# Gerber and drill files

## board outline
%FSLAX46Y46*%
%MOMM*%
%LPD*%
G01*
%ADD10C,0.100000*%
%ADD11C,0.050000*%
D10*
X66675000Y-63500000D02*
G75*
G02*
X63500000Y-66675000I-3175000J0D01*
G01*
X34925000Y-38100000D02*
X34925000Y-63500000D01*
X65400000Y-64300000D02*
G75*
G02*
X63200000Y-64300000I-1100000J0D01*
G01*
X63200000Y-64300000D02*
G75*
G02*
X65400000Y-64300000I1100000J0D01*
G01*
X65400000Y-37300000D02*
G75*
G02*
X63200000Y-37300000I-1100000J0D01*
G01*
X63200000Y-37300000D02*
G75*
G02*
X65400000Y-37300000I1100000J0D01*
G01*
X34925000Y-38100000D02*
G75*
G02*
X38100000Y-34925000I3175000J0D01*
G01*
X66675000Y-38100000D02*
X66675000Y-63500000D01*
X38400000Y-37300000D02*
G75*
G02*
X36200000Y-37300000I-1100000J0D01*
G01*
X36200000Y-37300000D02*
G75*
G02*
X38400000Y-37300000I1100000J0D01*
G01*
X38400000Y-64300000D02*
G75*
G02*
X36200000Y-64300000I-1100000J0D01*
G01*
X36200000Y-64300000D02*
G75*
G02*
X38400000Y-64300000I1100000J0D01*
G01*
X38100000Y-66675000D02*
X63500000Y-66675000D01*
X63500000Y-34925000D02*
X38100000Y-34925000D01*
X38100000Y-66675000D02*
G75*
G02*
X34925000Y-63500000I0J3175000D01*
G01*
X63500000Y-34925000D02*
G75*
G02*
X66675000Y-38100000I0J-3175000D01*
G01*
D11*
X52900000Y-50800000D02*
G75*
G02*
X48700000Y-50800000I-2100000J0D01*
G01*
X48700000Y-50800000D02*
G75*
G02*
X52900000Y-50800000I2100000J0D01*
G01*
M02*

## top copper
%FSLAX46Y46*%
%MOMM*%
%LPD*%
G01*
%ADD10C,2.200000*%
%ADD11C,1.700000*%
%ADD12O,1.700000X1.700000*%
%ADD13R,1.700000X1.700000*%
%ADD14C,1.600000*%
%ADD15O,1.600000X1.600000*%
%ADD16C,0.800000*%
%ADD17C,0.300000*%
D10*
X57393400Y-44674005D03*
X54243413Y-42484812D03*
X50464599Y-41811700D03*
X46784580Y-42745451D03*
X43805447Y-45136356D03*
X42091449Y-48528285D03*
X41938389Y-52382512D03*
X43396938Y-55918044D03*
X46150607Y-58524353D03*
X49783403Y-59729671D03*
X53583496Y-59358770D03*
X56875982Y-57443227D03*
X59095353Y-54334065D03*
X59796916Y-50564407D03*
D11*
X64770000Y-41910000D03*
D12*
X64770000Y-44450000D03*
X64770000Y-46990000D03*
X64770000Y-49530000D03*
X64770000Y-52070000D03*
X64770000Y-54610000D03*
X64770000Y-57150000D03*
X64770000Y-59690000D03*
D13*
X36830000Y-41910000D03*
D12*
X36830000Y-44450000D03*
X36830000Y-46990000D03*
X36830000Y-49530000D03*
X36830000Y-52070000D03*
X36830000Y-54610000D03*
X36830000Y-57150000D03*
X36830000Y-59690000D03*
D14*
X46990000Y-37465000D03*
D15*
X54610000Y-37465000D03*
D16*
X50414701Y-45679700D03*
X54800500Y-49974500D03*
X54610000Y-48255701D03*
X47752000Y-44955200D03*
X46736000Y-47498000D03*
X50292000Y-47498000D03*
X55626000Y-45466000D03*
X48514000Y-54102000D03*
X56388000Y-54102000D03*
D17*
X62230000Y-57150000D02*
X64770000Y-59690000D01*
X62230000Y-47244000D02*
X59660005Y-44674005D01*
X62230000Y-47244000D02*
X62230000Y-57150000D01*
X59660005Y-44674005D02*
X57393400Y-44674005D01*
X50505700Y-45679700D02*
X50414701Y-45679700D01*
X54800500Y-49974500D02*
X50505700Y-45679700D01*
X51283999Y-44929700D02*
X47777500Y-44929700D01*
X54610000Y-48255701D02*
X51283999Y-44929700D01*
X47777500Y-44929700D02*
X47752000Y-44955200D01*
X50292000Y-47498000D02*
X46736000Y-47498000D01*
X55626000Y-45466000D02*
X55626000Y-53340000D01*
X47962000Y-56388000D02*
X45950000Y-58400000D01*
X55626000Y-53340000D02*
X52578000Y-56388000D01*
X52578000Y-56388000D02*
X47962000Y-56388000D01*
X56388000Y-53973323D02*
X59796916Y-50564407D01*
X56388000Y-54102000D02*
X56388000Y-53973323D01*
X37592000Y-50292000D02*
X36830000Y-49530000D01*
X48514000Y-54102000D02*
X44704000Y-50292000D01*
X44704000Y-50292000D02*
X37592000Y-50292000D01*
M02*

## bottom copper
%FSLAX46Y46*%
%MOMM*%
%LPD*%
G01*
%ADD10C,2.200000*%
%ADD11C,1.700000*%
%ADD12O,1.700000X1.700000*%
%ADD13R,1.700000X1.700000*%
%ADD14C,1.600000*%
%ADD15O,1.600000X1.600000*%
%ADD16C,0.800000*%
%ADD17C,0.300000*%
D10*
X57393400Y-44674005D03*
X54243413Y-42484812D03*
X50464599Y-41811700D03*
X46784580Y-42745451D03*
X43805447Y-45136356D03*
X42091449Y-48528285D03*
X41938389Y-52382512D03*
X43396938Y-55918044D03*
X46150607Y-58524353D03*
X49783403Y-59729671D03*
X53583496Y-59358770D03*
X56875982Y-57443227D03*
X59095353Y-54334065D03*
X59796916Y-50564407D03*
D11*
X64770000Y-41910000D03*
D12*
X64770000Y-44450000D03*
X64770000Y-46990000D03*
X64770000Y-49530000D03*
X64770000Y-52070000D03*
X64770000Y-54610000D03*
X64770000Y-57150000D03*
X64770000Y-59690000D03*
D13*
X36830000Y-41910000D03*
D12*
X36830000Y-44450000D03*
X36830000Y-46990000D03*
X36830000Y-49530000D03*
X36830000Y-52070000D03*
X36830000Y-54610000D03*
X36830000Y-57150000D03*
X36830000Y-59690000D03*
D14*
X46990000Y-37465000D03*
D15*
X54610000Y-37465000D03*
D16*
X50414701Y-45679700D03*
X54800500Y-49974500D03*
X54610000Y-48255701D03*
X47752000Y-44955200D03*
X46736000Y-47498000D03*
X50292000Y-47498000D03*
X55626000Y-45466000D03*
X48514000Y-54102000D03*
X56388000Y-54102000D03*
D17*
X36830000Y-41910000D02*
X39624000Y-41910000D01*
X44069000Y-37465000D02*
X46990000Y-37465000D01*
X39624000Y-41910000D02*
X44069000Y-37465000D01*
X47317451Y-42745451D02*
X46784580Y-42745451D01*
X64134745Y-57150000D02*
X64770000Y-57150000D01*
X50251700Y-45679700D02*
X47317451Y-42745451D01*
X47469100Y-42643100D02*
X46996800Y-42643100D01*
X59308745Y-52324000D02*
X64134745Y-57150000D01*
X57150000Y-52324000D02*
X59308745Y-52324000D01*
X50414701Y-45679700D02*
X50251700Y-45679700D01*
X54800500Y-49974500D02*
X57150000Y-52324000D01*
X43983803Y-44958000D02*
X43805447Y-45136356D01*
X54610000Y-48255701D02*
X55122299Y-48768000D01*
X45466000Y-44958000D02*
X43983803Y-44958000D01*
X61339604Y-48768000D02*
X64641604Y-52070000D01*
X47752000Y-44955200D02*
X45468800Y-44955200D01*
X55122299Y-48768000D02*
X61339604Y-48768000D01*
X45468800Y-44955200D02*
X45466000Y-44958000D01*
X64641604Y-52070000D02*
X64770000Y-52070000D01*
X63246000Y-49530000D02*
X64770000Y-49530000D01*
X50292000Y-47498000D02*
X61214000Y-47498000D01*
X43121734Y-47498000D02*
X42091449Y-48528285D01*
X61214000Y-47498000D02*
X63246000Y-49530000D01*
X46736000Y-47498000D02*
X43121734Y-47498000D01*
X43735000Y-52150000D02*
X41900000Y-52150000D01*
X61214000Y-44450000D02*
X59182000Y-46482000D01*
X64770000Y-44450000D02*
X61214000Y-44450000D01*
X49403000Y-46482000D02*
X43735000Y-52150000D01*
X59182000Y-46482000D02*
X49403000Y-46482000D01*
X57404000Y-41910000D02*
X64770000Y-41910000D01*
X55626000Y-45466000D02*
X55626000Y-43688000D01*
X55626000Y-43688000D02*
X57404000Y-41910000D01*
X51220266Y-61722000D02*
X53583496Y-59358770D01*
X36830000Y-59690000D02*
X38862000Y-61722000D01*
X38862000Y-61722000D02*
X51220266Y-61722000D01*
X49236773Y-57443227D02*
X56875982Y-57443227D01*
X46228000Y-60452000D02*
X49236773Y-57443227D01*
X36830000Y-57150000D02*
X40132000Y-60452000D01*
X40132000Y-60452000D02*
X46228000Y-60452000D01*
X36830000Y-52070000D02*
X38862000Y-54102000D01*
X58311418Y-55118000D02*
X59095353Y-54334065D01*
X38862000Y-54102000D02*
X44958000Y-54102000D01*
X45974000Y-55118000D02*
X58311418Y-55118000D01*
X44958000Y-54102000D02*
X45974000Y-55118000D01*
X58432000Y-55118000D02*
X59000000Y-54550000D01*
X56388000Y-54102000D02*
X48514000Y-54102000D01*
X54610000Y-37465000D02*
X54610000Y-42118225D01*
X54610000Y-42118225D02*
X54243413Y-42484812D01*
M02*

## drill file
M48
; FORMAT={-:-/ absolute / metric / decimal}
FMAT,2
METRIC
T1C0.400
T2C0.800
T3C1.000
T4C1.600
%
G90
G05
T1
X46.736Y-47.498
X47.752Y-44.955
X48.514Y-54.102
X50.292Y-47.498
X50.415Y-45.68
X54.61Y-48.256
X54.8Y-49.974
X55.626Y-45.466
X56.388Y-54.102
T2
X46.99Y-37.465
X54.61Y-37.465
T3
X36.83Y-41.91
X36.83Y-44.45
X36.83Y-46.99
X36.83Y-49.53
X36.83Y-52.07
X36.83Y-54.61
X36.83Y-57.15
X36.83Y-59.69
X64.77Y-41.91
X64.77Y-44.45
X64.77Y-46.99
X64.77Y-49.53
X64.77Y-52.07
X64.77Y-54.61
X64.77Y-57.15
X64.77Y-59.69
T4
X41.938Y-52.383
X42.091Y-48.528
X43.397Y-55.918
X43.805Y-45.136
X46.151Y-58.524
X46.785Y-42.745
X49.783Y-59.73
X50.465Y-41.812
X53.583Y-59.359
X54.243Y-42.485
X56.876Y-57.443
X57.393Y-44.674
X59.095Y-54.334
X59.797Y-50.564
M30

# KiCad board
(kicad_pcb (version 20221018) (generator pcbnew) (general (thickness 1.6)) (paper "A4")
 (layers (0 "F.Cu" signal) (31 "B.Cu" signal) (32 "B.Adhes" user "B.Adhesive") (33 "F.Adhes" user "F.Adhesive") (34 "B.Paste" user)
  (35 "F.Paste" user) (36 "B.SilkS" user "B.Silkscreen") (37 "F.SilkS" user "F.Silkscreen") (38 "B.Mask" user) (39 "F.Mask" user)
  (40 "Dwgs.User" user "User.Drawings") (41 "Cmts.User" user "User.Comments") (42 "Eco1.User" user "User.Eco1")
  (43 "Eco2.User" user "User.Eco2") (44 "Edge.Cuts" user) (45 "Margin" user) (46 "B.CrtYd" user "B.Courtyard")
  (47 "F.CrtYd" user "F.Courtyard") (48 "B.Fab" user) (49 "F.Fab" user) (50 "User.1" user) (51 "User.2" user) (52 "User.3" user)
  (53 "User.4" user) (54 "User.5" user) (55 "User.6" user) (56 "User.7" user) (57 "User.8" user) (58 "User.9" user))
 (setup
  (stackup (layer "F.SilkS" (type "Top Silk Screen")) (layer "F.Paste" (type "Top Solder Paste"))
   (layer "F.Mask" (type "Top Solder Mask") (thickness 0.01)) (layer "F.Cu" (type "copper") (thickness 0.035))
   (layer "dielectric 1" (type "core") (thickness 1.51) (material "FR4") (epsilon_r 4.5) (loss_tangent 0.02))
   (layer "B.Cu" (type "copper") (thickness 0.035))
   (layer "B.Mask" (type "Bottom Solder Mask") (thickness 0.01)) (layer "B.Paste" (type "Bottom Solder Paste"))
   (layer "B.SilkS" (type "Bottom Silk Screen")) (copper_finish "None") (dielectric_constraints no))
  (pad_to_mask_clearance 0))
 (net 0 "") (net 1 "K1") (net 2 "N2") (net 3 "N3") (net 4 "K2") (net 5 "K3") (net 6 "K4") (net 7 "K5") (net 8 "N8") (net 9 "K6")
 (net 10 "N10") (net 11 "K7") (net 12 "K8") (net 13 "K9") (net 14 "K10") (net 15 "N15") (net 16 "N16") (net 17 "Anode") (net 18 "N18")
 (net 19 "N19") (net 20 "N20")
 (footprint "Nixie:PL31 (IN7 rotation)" (layer "F.Cu") (at 50.8 50.8 90)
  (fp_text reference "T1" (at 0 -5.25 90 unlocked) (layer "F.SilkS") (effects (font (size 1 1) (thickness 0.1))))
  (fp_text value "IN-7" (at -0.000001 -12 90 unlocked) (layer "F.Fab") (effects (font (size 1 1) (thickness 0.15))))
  (fp_circle (center 0 0) (end 2.1 0) (stroke (width 0.05) (type default)) (fill none) (layer "Edge.Cuts"))
  (pad "1" thru_hole circle (at 6.125995 6.5934 271.5) (size 2.2 2.2) (drill 1.6) (layers "*.Cu" "*.Mask") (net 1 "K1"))
  (pad "2" thru_hole circle (at 8.315188 3.443413 271.5) (size 2.2 2.2) (drill 1.6) (layers "*.Cu" "*.Mask") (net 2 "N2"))
  (pad "3" thru_hole circle (at 8.9883 -0.335401 271.5) (size 2.2 2.2) (drill 1.6) (layers "*.Cu" "*.Mask") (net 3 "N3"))
  (pad "4" thru_hole circle (at 8.054549 -4.01542 271.5) (size 2.2 2.2) (drill 1.6) (layers "*.Cu" "*.Mask") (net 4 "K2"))
  (pad "5" thru_hole circle (at 5.663644 -6.994553 271.5) (size 2.2 2.2) (drill 1.6) (layers "*.Cu" "*.Mask") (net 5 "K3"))
  (pad "6" thru_hole circle (at 2.271715 -8.708551 271.5) (size 2.2 2.2) (drill 1.6) (layers "*.Cu" "*.Mask") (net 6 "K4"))
  (pad "7" thru_hole circle (at -1.582512 -8.861611 271.5) (size 2.2 2.2) (drill 1.6) (layers "*.Cu" "*.Mask") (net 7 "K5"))
  (pad "8" thru_hole circle (at -5.118044 -7.403062 271.5) (size 2.2 2.2) (drill 1.6) (layers "*.Cu" "*.Mask") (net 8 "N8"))
  (pad "9" thru_hole circle (at -7.724353 -4.649393 271.5) (size 2.2 2.2) (drill 1.6) (layers "*.Cu" "*.Mask") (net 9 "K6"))
  (pad "10" thru_hole circle (at -8.929671 -1.016597 271.5) (size 2.2 2.2) (drill 1.6) (layers "*.Cu" "*.Mask") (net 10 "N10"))
  (pad "11" thru_hole circle (at -8.55877 2.783496 271.5) (size 2.2 2.2) (drill 1.6) (layers "*.Cu" "*.Mask") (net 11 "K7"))
  (pad "12" thru_hole circle (at -6.643227 6.075982 271.5) (size 2.2 2.2) (drill 1.6) (layers "*.Cu" "*.Mask") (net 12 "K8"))
  (pad "13" thru_hole circle (at -3.534065 8.295353 271.5) (size 2.2 2.2) (drill 1.6) (layers "*.Cu" "*.Mask") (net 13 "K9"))
  (pad "14" thru_hole circle (at 0.235593 8.996916 271.5) (size 2.2 2.2) (drill 1.6) (layers "*.Cu" "*.Mask") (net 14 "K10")))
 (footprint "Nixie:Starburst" (layer "F.Cu") (at 43 63.25)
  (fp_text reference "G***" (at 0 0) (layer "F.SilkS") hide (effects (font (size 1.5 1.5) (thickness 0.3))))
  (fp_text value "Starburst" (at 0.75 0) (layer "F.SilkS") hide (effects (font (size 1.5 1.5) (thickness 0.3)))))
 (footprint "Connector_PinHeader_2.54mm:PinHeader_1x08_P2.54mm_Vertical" (layer "B.Cu") (at 64.77 41.91 180)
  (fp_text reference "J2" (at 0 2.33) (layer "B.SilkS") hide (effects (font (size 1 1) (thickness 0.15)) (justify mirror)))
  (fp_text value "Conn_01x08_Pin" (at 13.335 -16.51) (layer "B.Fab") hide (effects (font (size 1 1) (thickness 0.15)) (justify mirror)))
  (pad "1" thru_hole circle (at 0 0 180) (size 1.7 1.7) (drill 1) (layers "*.Cu" "*.Mask") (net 9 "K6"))
  (pad "2" thru_hole oval (at 0 -2.54 180) (size 1.7 1.7) (drill 1) (layers "*.Cu" "*.Mask") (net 7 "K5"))
  (pad "3" thru_hole oval (at 0 -5.08 180) (size 1.7 1.7) (drill 1) (layers "*.Cu" "*.Mask") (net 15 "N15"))
  (pad "4" thru_hole oval (at 0 -7.62 180) (size 1.7 1.7) (drill 1) (layers "*.Cu" "*.Mask") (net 6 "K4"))
  (pad "5" thru_hole oval (at 0 -10.16 180) (size 1.7 1.7) (drill 1) (layers "*.Cu" "*.Mask") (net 5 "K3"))
  (pad "6" thru_hole oval (at 0 -12.7 180) (size 1.7 1.7) (drill 1) (layers "*.Cu" "*.Mask") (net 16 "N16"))
  (pad "7" thru_hole oval (at 0 -15.24 180) (size 1.7 1.7) (drill 1) (layers "*.Cu" "*.Mask") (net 4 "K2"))
  (pad "8" thru_hole oval (at 0 -17.78 180) (size 1.7 1.7) (drill 1) (layers "*.Cu" "*.Mask") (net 1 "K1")))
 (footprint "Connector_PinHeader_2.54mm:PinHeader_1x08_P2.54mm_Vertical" (layer "B.Cu") (at 36.83 41.91 180)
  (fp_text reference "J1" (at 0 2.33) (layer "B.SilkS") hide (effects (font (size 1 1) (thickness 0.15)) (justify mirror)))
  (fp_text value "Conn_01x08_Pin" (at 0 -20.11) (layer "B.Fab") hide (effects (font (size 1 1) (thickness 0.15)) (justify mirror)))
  (pad "1" thru_hole rect (at 0 0 180) (size 1.7 1.7) (drill 1) (layers "*.Cu" "*.Mask") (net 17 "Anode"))
  (pad "2" thru_hole oval (at 0 -2.54 180) (size 1.7 1.7) (drill 1) (layers "*.Cu" "*.Mask") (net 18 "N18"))
  (pad "3" thru_hole oval (at 0 -5.08 180) (size 1.7 1.7) (drill 1) (layers "*.Cu" "*.Mask") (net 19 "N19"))
  (pad "4" thru_hole oval (at 0 -7.62 180) (size 1.7 1.7) (drill 1) (layers "*.Cu" "*.Mask") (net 14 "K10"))
  (pad "5" thru_hole oval (at 0 -10.16 180) (size 1.7 1.7) (drill 1) (layers "*.Cu" "*.Mask") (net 13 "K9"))
  (pad "6" thru_hole oval (at 0 -12.7 180) (size 1.7 1.7) (drill 1) (layers "*.Cu" "*.Mask") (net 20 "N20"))
  (pad "7" thru_hole oval (at 0 -15.24 180) (size 1.7 1.7) (drill 1) (layers "*.Cu" "*.Mask") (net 12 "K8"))
  (pad "8" thru_hole oval (at 0 -17.78 180) (size 1.7 1.7) (drill 1) (layers "*.Cu" "*.Mask") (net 11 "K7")))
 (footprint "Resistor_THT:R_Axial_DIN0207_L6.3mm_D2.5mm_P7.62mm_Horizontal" (layer "B.Cu") (at 46.99 37.465)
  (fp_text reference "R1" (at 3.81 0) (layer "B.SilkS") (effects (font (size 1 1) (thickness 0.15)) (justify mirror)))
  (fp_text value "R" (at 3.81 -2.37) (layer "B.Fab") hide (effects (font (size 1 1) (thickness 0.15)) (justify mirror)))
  (pad "1" thru_hole circle (at 0 0) (size 1.6 1.6) (drill 0.8) (layers "*.Cu" "*.Mask") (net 17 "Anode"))
  (pad "2" thru_hole oval (at 7.62 0) (size 1.6 1.6) (drill 0.8) (layers "*.Cu" "*.Mask") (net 2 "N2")))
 (gr_arc (start 66.675 63.5) (mid 65.745064 65.745064) (end 63.5 66.675) (stroke (width 0.1) (type default)) (layer "Edge.Cuts"))
 (gr_line (start 34.925 38.1) (end 34.925 63.5) (stroke (width 0.1) (type default)) (layer "Edge.Cuts"))
 (gr_circle (center 64.3 64.3) (end 65.4 64.3) (stroke (width 0.1) (type default)) (fill none) (layer "Edge.Cuts"))
 (gr_circle (center 64.3 37.3) (end 65.4 37.3) (stroke (width 0.1) (type default)) (fill none) (layer "Edge.Cuts"))
 (gr_arc (start 34.925 38.1) (mid 35.854936 35.854936) (end 38.1 34.925) (stroke (width 0.1) (type default)) (layer "Edge.Cuts"))
 (gr_line (start 66.675 38.1) (end 66.675 63.5) (stroke (width 0.1) (type default)) (layer "Edge.Cuts"))
 (gr_circle (center 37.3 37.3) (end 38.4 37.3) (stroke (width 0.1) (type default)) (fill none) (layer "Edge.Cuts"))
 (gr_circle (center 37.3 64.3) (end 38.4 64.3) (stroke (width 0.1) (type default)) (fill none) (layer "Edge.Cuts"))
 (gr_line (start 38.1 66.675) (end 63.5 66.675) (stroke (width 0.1) (type default)) (layer "Edge.Cuts"))
 (gr_line (start 63.5 34.925) (end 38.1 34.925) (stroke (width 0.1) (type default)) (layer "Edge.Cuts"))
 (gr_arc (start 38.1 66.675) (mid 35.854936 65.745064) (end 34.925 63.5) (stroke (width 0.1) (type default)) (layer "Edge.Cuts"))
 (gr_arc (start 63.5 34.925) (mid 65.745064 35.854936) (end 66.675 38.1) (stroke (width 0.1) (type default)) (layer "Edge.Cuts"))
 (segment (start 36.83 41.91) (end 39.624 41.91) (width 0.3) (layer "B.Cu") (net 17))
 (segment (start 44.069 37.465) (end 46.99 37.465) (width 0.3) (layer "B.Cu") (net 17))
 (segment (start 39.624 41.91) (end 44.069 37.465) (width 0.3) (layer "B.Cu") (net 17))
 (segment (start 62.23 57.15) (end 64.77 59.69) (width 0.3) (layer "F.Cu") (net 1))
 (segment (start 62.23 47.244) (end 59.660005 44.674005) (width 0.3) (layer "F.Cu") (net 1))
 (segment (start 62.23 47.244) (end 62.23 57.15) (width 0.3) (layer "F.Cu") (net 1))
 (segment (start 59.660005 44.674005) (end 57.3934 44.674005) (width 0.3) (layer "F.Cu") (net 1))
 (segment (start 50.5057 45.6797) (end 50.414701 45.6797) (width 0.3) (layer "F.Cu") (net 4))
 (segment (start 54.8005 49.9745) (end 50.5057 45.6797) (width 0.3) (layer "F.Cu") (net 4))
 (via (at 50.414701 45.6797) (size 0.8) (drill 0.4) (layers "F.Cu" "B.Cu") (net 4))
 (via (at 54.8005 49.9745) (size 0.8) (drill 0.4) (layers "F.Cu" "B.Cu") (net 4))
 (segment (start 47.317451 42.745451) (end 46.78458 42.745451) (width 0.3) (layer "B.Cu") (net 4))
 (segment (start 64.134745 57.15) (end 64.77 57.15) (width 0.3) (layer "B.Cu") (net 4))
 (segment (start 50.2517 45.6797) (end 47.317451 42.745451) (width 0.3) (layer "B.Cu") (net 4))
 (segment (start 47.4691 42.6431) (end 46.9968 42.6431) (width 0.3) (layer "B.Cu") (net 4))
 (segment (start 59.308745 52.324) (end 64.134745 57.15) (width 0.3) (layer "B.Cu") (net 4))
 (segment (start 57.15 52.324) (end 59.308745 52.324) (width 0.3) (layer "B.Cu") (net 4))
 (segment (start 50.414701 45.6797) (end 50.2517 45.6797) (width 0.3) (layer "B.Cu") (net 4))
 (segment (start 54.8005 49.9745) (end 57.15 52.324) (width 0.3) (layer "B.Cu") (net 4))
 (segment (start 51.283999 44.9297) (end 47.7775 44.9297) (width 0.3) (layer "F.Cu") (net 5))
 (segment (start 54.61 48.255701) (end 51.283999 44.9297) (width 0.3) (layer "F.Cu") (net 5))
 (segment (start 47.7775 44.9297) (end 47.752 44.9552) (width 0.3) (layer "F.Cu") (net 5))
 (via (at 54.61 48.255701) (size 0.8) (drill 0.4) (layers "F.Cu" "B.Cu") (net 5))
 (via (at 47.752 44.9552) (size 0.8) (drill 0.4) (layers "F.Cu" "B.Cu") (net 5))
 (segment (start 43.983803 44.958) (end 43.805447 45.136356) (width 0.3) (layer "B.Cu") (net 5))
 (segment (start 54.61 48.255701) (end 55.122299 48.768) (width 0.3) (layer "B.Cu") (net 5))
 (segment (start 45.466 44.958) (end 43.983803 44.958) (width 0.3) (layer "B.Cu") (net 5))
 (segment (start 61.339604 48.768) (end 64.641604 52.07) (width 0.3) (layer "B.Cu") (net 5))
 (segment (start 47.752 44.9552) (end 45.4688 44.9552) (width 0.3) (layer "B.Cu") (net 5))
 (segment (start 55.122299 48.768) (end 61.339604 48.768) (width 0.3) (layer "B.Cu") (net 5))
 (segment (start 45.4688 44.9552) (end 45.466 44.958) (width 0.3) (layer "B.Cu") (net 5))
 (segment (start 64.641604 52.07) (end 64.77 52.07) (width 0.3) (layer "B.Cu") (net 5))
 (segment (start 50.292 47.498) (end 46.736 47.498) (width 0.3) (layer "F.Cu") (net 6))
 (via (at 46.736 47.498) (size 0.8) (drill 0.4) (layers "F.Cu" "B.Cu") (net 6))
 (via (at 50.292 47.498) (size 0.8) (drill 0.4) (layers "F.Cu" "B.Cu") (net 6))
 (segment (start 63.246 49.53) (end 64.77 49.53) (width 0.3) (layer "B.Cu") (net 6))
 (segment (start 50.292 47.498) (end 61.214 47.498) (width 0.3) (layer "B.Cu") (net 6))
 (segment (start 43.121734 47.498) (end 42.091449 48.528285) (width 0.3) (layer "B.Cu") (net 6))
 (segment (start 61.214 47.498) (end 63.246 49.53) (width 0.3) (layer "B.Cu") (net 6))
 (segment (start 46.736 47.498) (end 43.121734 47.498) (width 0.3) (layer "B.Cu") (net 6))
 (segment (start 43.735 52.15) (end 41.9 52.15) (width 0.3) (layer "B.Cu") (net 7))
 (segment (start 61.214 44.45) (end 59.182 46.482) (width 0.3) (layer "B.Cu") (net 7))
 (segment (start 64.77 44.45) (end 61.214 44.45) (width 0.3) (layer "B.Cu") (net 7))
 (segment (start 49.403 46.482) (end 43.735 52.15) (width 0.3) (layer "B.Cu") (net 7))
 (segment (start 59.182 46.482) (end 49.403 46.482) (width 0.3) (layer "B.Cu") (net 7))
 (segment (start 55.626 45.466) (end 55.626 53.34) (width 0.3) (layer "F.Cu") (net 9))
 (segment (start 47.962 56.388) (end 45.95 58.4) (width 0.3) (layer "F.Cu") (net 9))
 (segment (start 55.626 53.34) (end 52.578 56.388) (width 0.3) (layer "F.Cu") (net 9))
 (segment (start 52.578 56.388) (end 47.962 56.388) (width 0.3) (layer "F.Cu") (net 9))
 (via (at 55.626 45.466) (size 0.8) (drill 0.4) (layers "F.Cu" "B.Cu") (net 9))
 (segment (start 57.404 41.91) (end 64.77 41.91) (width 0.3) (layer "B.Cu") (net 9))
 (segment (start 55.626 45.466) (end 55.626 43.688) (width 0.3) (layer "B.Cu") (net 9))
 (segment (start 55.626 43.688) (end 57.404 41.91) (width 0.3) (layer "B.Cu") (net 9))
 (segment (start 51.220266 61.722) (end 53.583496 59.35877) (width 0.3) (layer "B.Cu") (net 11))
 (segment (start 36.83 59.69) (end 38.862 61.722) (width 0.3) (layer "B.Cu") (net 11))
 (segment (start 38.862 61.722) (end 51.220266 61.722) (width 0.3) (layer "B.Cu") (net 11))
 (segment (start 49.236773 57.443227) (end 56.875982 57.443227) (width 0.3) (layer "B.Cu") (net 12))
 (segment (start 46.228 60.452) (end 49.236773 57.443227) (width 0.3) (layer "B.Cu") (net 12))
 (segment (start 36.83 57.15) (end 40.132 60.452) (width 0.3) (layer "B.Cu") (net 12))
 (segment (start 40.132 60.452) (end 46.228 60.452) (width 0.3) (layer "B.Cu") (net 12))
 (segment (start 36.83 52.07) (end 38.862 54.102) (width 0.3) (layer "B.Cu") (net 13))
 (segment (start 58.311418 55.118) (end 59.095353 54.334065) (width 0.3) (layer "B.Cu") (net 13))
 (segment (start 38.862 54.102) (end 44.958 54.102) (width 0.3) (layer "B.Cu") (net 13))
 (segment (start 45.974 55.118) (end 58.311418 55.118) (width 0.3) (layer "B.Cu") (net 13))
 (segment (start 44.958 54.102) (end 45.974 55.118) (width 0.3) (layer "B.Cu") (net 13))
 (segment (start 58.432 55.118) (end 59 54.55) (width 0.3) (layer "B.Cu") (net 13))
 (segment (start 56.388 53.973323) (end 59.796916 50.564407) (width 0.3) (layer "F.Cu") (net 14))
 (segment (start 56.388 54.102) (end 56.388 53.973323) (width 0.3) (layer "F.Cu") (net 14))
 (segment (start 37.592 50.292) (end 36.83 49.53) (width 0.3) (layer "F.Cu") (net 14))
 (segment (start 48.514 54.102) (end 44.704 50.292) (width 0.3) (layer "F.Cu") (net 14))
 (segment (start 44.704 50.292) (end 37.592 50.292) (width 0.3) (layer "F.Cu") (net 14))
 (via (at 48.514 54.102) (size 0.8) (drill 0.4) (layers "F.Cu" "B.Cu") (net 14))
 (via (at 56.388 54.102) (size 0.8) (drill 0.4) (layers "F.Cu" "B.Cu") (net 14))
 (segment (start 56.388 54.102) (end 48.514 54.102) (width 0.3) (layer "B.Cu") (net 14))
 (segment (start 54.61 37.465) (end 54.61 42.118225) (width 0.3) (layer "B.Cu") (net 2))
 (segment (start 54.61 42.118225) (end 54.243413 42.484812) (width 0.3) (layer "B.Cu") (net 2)))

